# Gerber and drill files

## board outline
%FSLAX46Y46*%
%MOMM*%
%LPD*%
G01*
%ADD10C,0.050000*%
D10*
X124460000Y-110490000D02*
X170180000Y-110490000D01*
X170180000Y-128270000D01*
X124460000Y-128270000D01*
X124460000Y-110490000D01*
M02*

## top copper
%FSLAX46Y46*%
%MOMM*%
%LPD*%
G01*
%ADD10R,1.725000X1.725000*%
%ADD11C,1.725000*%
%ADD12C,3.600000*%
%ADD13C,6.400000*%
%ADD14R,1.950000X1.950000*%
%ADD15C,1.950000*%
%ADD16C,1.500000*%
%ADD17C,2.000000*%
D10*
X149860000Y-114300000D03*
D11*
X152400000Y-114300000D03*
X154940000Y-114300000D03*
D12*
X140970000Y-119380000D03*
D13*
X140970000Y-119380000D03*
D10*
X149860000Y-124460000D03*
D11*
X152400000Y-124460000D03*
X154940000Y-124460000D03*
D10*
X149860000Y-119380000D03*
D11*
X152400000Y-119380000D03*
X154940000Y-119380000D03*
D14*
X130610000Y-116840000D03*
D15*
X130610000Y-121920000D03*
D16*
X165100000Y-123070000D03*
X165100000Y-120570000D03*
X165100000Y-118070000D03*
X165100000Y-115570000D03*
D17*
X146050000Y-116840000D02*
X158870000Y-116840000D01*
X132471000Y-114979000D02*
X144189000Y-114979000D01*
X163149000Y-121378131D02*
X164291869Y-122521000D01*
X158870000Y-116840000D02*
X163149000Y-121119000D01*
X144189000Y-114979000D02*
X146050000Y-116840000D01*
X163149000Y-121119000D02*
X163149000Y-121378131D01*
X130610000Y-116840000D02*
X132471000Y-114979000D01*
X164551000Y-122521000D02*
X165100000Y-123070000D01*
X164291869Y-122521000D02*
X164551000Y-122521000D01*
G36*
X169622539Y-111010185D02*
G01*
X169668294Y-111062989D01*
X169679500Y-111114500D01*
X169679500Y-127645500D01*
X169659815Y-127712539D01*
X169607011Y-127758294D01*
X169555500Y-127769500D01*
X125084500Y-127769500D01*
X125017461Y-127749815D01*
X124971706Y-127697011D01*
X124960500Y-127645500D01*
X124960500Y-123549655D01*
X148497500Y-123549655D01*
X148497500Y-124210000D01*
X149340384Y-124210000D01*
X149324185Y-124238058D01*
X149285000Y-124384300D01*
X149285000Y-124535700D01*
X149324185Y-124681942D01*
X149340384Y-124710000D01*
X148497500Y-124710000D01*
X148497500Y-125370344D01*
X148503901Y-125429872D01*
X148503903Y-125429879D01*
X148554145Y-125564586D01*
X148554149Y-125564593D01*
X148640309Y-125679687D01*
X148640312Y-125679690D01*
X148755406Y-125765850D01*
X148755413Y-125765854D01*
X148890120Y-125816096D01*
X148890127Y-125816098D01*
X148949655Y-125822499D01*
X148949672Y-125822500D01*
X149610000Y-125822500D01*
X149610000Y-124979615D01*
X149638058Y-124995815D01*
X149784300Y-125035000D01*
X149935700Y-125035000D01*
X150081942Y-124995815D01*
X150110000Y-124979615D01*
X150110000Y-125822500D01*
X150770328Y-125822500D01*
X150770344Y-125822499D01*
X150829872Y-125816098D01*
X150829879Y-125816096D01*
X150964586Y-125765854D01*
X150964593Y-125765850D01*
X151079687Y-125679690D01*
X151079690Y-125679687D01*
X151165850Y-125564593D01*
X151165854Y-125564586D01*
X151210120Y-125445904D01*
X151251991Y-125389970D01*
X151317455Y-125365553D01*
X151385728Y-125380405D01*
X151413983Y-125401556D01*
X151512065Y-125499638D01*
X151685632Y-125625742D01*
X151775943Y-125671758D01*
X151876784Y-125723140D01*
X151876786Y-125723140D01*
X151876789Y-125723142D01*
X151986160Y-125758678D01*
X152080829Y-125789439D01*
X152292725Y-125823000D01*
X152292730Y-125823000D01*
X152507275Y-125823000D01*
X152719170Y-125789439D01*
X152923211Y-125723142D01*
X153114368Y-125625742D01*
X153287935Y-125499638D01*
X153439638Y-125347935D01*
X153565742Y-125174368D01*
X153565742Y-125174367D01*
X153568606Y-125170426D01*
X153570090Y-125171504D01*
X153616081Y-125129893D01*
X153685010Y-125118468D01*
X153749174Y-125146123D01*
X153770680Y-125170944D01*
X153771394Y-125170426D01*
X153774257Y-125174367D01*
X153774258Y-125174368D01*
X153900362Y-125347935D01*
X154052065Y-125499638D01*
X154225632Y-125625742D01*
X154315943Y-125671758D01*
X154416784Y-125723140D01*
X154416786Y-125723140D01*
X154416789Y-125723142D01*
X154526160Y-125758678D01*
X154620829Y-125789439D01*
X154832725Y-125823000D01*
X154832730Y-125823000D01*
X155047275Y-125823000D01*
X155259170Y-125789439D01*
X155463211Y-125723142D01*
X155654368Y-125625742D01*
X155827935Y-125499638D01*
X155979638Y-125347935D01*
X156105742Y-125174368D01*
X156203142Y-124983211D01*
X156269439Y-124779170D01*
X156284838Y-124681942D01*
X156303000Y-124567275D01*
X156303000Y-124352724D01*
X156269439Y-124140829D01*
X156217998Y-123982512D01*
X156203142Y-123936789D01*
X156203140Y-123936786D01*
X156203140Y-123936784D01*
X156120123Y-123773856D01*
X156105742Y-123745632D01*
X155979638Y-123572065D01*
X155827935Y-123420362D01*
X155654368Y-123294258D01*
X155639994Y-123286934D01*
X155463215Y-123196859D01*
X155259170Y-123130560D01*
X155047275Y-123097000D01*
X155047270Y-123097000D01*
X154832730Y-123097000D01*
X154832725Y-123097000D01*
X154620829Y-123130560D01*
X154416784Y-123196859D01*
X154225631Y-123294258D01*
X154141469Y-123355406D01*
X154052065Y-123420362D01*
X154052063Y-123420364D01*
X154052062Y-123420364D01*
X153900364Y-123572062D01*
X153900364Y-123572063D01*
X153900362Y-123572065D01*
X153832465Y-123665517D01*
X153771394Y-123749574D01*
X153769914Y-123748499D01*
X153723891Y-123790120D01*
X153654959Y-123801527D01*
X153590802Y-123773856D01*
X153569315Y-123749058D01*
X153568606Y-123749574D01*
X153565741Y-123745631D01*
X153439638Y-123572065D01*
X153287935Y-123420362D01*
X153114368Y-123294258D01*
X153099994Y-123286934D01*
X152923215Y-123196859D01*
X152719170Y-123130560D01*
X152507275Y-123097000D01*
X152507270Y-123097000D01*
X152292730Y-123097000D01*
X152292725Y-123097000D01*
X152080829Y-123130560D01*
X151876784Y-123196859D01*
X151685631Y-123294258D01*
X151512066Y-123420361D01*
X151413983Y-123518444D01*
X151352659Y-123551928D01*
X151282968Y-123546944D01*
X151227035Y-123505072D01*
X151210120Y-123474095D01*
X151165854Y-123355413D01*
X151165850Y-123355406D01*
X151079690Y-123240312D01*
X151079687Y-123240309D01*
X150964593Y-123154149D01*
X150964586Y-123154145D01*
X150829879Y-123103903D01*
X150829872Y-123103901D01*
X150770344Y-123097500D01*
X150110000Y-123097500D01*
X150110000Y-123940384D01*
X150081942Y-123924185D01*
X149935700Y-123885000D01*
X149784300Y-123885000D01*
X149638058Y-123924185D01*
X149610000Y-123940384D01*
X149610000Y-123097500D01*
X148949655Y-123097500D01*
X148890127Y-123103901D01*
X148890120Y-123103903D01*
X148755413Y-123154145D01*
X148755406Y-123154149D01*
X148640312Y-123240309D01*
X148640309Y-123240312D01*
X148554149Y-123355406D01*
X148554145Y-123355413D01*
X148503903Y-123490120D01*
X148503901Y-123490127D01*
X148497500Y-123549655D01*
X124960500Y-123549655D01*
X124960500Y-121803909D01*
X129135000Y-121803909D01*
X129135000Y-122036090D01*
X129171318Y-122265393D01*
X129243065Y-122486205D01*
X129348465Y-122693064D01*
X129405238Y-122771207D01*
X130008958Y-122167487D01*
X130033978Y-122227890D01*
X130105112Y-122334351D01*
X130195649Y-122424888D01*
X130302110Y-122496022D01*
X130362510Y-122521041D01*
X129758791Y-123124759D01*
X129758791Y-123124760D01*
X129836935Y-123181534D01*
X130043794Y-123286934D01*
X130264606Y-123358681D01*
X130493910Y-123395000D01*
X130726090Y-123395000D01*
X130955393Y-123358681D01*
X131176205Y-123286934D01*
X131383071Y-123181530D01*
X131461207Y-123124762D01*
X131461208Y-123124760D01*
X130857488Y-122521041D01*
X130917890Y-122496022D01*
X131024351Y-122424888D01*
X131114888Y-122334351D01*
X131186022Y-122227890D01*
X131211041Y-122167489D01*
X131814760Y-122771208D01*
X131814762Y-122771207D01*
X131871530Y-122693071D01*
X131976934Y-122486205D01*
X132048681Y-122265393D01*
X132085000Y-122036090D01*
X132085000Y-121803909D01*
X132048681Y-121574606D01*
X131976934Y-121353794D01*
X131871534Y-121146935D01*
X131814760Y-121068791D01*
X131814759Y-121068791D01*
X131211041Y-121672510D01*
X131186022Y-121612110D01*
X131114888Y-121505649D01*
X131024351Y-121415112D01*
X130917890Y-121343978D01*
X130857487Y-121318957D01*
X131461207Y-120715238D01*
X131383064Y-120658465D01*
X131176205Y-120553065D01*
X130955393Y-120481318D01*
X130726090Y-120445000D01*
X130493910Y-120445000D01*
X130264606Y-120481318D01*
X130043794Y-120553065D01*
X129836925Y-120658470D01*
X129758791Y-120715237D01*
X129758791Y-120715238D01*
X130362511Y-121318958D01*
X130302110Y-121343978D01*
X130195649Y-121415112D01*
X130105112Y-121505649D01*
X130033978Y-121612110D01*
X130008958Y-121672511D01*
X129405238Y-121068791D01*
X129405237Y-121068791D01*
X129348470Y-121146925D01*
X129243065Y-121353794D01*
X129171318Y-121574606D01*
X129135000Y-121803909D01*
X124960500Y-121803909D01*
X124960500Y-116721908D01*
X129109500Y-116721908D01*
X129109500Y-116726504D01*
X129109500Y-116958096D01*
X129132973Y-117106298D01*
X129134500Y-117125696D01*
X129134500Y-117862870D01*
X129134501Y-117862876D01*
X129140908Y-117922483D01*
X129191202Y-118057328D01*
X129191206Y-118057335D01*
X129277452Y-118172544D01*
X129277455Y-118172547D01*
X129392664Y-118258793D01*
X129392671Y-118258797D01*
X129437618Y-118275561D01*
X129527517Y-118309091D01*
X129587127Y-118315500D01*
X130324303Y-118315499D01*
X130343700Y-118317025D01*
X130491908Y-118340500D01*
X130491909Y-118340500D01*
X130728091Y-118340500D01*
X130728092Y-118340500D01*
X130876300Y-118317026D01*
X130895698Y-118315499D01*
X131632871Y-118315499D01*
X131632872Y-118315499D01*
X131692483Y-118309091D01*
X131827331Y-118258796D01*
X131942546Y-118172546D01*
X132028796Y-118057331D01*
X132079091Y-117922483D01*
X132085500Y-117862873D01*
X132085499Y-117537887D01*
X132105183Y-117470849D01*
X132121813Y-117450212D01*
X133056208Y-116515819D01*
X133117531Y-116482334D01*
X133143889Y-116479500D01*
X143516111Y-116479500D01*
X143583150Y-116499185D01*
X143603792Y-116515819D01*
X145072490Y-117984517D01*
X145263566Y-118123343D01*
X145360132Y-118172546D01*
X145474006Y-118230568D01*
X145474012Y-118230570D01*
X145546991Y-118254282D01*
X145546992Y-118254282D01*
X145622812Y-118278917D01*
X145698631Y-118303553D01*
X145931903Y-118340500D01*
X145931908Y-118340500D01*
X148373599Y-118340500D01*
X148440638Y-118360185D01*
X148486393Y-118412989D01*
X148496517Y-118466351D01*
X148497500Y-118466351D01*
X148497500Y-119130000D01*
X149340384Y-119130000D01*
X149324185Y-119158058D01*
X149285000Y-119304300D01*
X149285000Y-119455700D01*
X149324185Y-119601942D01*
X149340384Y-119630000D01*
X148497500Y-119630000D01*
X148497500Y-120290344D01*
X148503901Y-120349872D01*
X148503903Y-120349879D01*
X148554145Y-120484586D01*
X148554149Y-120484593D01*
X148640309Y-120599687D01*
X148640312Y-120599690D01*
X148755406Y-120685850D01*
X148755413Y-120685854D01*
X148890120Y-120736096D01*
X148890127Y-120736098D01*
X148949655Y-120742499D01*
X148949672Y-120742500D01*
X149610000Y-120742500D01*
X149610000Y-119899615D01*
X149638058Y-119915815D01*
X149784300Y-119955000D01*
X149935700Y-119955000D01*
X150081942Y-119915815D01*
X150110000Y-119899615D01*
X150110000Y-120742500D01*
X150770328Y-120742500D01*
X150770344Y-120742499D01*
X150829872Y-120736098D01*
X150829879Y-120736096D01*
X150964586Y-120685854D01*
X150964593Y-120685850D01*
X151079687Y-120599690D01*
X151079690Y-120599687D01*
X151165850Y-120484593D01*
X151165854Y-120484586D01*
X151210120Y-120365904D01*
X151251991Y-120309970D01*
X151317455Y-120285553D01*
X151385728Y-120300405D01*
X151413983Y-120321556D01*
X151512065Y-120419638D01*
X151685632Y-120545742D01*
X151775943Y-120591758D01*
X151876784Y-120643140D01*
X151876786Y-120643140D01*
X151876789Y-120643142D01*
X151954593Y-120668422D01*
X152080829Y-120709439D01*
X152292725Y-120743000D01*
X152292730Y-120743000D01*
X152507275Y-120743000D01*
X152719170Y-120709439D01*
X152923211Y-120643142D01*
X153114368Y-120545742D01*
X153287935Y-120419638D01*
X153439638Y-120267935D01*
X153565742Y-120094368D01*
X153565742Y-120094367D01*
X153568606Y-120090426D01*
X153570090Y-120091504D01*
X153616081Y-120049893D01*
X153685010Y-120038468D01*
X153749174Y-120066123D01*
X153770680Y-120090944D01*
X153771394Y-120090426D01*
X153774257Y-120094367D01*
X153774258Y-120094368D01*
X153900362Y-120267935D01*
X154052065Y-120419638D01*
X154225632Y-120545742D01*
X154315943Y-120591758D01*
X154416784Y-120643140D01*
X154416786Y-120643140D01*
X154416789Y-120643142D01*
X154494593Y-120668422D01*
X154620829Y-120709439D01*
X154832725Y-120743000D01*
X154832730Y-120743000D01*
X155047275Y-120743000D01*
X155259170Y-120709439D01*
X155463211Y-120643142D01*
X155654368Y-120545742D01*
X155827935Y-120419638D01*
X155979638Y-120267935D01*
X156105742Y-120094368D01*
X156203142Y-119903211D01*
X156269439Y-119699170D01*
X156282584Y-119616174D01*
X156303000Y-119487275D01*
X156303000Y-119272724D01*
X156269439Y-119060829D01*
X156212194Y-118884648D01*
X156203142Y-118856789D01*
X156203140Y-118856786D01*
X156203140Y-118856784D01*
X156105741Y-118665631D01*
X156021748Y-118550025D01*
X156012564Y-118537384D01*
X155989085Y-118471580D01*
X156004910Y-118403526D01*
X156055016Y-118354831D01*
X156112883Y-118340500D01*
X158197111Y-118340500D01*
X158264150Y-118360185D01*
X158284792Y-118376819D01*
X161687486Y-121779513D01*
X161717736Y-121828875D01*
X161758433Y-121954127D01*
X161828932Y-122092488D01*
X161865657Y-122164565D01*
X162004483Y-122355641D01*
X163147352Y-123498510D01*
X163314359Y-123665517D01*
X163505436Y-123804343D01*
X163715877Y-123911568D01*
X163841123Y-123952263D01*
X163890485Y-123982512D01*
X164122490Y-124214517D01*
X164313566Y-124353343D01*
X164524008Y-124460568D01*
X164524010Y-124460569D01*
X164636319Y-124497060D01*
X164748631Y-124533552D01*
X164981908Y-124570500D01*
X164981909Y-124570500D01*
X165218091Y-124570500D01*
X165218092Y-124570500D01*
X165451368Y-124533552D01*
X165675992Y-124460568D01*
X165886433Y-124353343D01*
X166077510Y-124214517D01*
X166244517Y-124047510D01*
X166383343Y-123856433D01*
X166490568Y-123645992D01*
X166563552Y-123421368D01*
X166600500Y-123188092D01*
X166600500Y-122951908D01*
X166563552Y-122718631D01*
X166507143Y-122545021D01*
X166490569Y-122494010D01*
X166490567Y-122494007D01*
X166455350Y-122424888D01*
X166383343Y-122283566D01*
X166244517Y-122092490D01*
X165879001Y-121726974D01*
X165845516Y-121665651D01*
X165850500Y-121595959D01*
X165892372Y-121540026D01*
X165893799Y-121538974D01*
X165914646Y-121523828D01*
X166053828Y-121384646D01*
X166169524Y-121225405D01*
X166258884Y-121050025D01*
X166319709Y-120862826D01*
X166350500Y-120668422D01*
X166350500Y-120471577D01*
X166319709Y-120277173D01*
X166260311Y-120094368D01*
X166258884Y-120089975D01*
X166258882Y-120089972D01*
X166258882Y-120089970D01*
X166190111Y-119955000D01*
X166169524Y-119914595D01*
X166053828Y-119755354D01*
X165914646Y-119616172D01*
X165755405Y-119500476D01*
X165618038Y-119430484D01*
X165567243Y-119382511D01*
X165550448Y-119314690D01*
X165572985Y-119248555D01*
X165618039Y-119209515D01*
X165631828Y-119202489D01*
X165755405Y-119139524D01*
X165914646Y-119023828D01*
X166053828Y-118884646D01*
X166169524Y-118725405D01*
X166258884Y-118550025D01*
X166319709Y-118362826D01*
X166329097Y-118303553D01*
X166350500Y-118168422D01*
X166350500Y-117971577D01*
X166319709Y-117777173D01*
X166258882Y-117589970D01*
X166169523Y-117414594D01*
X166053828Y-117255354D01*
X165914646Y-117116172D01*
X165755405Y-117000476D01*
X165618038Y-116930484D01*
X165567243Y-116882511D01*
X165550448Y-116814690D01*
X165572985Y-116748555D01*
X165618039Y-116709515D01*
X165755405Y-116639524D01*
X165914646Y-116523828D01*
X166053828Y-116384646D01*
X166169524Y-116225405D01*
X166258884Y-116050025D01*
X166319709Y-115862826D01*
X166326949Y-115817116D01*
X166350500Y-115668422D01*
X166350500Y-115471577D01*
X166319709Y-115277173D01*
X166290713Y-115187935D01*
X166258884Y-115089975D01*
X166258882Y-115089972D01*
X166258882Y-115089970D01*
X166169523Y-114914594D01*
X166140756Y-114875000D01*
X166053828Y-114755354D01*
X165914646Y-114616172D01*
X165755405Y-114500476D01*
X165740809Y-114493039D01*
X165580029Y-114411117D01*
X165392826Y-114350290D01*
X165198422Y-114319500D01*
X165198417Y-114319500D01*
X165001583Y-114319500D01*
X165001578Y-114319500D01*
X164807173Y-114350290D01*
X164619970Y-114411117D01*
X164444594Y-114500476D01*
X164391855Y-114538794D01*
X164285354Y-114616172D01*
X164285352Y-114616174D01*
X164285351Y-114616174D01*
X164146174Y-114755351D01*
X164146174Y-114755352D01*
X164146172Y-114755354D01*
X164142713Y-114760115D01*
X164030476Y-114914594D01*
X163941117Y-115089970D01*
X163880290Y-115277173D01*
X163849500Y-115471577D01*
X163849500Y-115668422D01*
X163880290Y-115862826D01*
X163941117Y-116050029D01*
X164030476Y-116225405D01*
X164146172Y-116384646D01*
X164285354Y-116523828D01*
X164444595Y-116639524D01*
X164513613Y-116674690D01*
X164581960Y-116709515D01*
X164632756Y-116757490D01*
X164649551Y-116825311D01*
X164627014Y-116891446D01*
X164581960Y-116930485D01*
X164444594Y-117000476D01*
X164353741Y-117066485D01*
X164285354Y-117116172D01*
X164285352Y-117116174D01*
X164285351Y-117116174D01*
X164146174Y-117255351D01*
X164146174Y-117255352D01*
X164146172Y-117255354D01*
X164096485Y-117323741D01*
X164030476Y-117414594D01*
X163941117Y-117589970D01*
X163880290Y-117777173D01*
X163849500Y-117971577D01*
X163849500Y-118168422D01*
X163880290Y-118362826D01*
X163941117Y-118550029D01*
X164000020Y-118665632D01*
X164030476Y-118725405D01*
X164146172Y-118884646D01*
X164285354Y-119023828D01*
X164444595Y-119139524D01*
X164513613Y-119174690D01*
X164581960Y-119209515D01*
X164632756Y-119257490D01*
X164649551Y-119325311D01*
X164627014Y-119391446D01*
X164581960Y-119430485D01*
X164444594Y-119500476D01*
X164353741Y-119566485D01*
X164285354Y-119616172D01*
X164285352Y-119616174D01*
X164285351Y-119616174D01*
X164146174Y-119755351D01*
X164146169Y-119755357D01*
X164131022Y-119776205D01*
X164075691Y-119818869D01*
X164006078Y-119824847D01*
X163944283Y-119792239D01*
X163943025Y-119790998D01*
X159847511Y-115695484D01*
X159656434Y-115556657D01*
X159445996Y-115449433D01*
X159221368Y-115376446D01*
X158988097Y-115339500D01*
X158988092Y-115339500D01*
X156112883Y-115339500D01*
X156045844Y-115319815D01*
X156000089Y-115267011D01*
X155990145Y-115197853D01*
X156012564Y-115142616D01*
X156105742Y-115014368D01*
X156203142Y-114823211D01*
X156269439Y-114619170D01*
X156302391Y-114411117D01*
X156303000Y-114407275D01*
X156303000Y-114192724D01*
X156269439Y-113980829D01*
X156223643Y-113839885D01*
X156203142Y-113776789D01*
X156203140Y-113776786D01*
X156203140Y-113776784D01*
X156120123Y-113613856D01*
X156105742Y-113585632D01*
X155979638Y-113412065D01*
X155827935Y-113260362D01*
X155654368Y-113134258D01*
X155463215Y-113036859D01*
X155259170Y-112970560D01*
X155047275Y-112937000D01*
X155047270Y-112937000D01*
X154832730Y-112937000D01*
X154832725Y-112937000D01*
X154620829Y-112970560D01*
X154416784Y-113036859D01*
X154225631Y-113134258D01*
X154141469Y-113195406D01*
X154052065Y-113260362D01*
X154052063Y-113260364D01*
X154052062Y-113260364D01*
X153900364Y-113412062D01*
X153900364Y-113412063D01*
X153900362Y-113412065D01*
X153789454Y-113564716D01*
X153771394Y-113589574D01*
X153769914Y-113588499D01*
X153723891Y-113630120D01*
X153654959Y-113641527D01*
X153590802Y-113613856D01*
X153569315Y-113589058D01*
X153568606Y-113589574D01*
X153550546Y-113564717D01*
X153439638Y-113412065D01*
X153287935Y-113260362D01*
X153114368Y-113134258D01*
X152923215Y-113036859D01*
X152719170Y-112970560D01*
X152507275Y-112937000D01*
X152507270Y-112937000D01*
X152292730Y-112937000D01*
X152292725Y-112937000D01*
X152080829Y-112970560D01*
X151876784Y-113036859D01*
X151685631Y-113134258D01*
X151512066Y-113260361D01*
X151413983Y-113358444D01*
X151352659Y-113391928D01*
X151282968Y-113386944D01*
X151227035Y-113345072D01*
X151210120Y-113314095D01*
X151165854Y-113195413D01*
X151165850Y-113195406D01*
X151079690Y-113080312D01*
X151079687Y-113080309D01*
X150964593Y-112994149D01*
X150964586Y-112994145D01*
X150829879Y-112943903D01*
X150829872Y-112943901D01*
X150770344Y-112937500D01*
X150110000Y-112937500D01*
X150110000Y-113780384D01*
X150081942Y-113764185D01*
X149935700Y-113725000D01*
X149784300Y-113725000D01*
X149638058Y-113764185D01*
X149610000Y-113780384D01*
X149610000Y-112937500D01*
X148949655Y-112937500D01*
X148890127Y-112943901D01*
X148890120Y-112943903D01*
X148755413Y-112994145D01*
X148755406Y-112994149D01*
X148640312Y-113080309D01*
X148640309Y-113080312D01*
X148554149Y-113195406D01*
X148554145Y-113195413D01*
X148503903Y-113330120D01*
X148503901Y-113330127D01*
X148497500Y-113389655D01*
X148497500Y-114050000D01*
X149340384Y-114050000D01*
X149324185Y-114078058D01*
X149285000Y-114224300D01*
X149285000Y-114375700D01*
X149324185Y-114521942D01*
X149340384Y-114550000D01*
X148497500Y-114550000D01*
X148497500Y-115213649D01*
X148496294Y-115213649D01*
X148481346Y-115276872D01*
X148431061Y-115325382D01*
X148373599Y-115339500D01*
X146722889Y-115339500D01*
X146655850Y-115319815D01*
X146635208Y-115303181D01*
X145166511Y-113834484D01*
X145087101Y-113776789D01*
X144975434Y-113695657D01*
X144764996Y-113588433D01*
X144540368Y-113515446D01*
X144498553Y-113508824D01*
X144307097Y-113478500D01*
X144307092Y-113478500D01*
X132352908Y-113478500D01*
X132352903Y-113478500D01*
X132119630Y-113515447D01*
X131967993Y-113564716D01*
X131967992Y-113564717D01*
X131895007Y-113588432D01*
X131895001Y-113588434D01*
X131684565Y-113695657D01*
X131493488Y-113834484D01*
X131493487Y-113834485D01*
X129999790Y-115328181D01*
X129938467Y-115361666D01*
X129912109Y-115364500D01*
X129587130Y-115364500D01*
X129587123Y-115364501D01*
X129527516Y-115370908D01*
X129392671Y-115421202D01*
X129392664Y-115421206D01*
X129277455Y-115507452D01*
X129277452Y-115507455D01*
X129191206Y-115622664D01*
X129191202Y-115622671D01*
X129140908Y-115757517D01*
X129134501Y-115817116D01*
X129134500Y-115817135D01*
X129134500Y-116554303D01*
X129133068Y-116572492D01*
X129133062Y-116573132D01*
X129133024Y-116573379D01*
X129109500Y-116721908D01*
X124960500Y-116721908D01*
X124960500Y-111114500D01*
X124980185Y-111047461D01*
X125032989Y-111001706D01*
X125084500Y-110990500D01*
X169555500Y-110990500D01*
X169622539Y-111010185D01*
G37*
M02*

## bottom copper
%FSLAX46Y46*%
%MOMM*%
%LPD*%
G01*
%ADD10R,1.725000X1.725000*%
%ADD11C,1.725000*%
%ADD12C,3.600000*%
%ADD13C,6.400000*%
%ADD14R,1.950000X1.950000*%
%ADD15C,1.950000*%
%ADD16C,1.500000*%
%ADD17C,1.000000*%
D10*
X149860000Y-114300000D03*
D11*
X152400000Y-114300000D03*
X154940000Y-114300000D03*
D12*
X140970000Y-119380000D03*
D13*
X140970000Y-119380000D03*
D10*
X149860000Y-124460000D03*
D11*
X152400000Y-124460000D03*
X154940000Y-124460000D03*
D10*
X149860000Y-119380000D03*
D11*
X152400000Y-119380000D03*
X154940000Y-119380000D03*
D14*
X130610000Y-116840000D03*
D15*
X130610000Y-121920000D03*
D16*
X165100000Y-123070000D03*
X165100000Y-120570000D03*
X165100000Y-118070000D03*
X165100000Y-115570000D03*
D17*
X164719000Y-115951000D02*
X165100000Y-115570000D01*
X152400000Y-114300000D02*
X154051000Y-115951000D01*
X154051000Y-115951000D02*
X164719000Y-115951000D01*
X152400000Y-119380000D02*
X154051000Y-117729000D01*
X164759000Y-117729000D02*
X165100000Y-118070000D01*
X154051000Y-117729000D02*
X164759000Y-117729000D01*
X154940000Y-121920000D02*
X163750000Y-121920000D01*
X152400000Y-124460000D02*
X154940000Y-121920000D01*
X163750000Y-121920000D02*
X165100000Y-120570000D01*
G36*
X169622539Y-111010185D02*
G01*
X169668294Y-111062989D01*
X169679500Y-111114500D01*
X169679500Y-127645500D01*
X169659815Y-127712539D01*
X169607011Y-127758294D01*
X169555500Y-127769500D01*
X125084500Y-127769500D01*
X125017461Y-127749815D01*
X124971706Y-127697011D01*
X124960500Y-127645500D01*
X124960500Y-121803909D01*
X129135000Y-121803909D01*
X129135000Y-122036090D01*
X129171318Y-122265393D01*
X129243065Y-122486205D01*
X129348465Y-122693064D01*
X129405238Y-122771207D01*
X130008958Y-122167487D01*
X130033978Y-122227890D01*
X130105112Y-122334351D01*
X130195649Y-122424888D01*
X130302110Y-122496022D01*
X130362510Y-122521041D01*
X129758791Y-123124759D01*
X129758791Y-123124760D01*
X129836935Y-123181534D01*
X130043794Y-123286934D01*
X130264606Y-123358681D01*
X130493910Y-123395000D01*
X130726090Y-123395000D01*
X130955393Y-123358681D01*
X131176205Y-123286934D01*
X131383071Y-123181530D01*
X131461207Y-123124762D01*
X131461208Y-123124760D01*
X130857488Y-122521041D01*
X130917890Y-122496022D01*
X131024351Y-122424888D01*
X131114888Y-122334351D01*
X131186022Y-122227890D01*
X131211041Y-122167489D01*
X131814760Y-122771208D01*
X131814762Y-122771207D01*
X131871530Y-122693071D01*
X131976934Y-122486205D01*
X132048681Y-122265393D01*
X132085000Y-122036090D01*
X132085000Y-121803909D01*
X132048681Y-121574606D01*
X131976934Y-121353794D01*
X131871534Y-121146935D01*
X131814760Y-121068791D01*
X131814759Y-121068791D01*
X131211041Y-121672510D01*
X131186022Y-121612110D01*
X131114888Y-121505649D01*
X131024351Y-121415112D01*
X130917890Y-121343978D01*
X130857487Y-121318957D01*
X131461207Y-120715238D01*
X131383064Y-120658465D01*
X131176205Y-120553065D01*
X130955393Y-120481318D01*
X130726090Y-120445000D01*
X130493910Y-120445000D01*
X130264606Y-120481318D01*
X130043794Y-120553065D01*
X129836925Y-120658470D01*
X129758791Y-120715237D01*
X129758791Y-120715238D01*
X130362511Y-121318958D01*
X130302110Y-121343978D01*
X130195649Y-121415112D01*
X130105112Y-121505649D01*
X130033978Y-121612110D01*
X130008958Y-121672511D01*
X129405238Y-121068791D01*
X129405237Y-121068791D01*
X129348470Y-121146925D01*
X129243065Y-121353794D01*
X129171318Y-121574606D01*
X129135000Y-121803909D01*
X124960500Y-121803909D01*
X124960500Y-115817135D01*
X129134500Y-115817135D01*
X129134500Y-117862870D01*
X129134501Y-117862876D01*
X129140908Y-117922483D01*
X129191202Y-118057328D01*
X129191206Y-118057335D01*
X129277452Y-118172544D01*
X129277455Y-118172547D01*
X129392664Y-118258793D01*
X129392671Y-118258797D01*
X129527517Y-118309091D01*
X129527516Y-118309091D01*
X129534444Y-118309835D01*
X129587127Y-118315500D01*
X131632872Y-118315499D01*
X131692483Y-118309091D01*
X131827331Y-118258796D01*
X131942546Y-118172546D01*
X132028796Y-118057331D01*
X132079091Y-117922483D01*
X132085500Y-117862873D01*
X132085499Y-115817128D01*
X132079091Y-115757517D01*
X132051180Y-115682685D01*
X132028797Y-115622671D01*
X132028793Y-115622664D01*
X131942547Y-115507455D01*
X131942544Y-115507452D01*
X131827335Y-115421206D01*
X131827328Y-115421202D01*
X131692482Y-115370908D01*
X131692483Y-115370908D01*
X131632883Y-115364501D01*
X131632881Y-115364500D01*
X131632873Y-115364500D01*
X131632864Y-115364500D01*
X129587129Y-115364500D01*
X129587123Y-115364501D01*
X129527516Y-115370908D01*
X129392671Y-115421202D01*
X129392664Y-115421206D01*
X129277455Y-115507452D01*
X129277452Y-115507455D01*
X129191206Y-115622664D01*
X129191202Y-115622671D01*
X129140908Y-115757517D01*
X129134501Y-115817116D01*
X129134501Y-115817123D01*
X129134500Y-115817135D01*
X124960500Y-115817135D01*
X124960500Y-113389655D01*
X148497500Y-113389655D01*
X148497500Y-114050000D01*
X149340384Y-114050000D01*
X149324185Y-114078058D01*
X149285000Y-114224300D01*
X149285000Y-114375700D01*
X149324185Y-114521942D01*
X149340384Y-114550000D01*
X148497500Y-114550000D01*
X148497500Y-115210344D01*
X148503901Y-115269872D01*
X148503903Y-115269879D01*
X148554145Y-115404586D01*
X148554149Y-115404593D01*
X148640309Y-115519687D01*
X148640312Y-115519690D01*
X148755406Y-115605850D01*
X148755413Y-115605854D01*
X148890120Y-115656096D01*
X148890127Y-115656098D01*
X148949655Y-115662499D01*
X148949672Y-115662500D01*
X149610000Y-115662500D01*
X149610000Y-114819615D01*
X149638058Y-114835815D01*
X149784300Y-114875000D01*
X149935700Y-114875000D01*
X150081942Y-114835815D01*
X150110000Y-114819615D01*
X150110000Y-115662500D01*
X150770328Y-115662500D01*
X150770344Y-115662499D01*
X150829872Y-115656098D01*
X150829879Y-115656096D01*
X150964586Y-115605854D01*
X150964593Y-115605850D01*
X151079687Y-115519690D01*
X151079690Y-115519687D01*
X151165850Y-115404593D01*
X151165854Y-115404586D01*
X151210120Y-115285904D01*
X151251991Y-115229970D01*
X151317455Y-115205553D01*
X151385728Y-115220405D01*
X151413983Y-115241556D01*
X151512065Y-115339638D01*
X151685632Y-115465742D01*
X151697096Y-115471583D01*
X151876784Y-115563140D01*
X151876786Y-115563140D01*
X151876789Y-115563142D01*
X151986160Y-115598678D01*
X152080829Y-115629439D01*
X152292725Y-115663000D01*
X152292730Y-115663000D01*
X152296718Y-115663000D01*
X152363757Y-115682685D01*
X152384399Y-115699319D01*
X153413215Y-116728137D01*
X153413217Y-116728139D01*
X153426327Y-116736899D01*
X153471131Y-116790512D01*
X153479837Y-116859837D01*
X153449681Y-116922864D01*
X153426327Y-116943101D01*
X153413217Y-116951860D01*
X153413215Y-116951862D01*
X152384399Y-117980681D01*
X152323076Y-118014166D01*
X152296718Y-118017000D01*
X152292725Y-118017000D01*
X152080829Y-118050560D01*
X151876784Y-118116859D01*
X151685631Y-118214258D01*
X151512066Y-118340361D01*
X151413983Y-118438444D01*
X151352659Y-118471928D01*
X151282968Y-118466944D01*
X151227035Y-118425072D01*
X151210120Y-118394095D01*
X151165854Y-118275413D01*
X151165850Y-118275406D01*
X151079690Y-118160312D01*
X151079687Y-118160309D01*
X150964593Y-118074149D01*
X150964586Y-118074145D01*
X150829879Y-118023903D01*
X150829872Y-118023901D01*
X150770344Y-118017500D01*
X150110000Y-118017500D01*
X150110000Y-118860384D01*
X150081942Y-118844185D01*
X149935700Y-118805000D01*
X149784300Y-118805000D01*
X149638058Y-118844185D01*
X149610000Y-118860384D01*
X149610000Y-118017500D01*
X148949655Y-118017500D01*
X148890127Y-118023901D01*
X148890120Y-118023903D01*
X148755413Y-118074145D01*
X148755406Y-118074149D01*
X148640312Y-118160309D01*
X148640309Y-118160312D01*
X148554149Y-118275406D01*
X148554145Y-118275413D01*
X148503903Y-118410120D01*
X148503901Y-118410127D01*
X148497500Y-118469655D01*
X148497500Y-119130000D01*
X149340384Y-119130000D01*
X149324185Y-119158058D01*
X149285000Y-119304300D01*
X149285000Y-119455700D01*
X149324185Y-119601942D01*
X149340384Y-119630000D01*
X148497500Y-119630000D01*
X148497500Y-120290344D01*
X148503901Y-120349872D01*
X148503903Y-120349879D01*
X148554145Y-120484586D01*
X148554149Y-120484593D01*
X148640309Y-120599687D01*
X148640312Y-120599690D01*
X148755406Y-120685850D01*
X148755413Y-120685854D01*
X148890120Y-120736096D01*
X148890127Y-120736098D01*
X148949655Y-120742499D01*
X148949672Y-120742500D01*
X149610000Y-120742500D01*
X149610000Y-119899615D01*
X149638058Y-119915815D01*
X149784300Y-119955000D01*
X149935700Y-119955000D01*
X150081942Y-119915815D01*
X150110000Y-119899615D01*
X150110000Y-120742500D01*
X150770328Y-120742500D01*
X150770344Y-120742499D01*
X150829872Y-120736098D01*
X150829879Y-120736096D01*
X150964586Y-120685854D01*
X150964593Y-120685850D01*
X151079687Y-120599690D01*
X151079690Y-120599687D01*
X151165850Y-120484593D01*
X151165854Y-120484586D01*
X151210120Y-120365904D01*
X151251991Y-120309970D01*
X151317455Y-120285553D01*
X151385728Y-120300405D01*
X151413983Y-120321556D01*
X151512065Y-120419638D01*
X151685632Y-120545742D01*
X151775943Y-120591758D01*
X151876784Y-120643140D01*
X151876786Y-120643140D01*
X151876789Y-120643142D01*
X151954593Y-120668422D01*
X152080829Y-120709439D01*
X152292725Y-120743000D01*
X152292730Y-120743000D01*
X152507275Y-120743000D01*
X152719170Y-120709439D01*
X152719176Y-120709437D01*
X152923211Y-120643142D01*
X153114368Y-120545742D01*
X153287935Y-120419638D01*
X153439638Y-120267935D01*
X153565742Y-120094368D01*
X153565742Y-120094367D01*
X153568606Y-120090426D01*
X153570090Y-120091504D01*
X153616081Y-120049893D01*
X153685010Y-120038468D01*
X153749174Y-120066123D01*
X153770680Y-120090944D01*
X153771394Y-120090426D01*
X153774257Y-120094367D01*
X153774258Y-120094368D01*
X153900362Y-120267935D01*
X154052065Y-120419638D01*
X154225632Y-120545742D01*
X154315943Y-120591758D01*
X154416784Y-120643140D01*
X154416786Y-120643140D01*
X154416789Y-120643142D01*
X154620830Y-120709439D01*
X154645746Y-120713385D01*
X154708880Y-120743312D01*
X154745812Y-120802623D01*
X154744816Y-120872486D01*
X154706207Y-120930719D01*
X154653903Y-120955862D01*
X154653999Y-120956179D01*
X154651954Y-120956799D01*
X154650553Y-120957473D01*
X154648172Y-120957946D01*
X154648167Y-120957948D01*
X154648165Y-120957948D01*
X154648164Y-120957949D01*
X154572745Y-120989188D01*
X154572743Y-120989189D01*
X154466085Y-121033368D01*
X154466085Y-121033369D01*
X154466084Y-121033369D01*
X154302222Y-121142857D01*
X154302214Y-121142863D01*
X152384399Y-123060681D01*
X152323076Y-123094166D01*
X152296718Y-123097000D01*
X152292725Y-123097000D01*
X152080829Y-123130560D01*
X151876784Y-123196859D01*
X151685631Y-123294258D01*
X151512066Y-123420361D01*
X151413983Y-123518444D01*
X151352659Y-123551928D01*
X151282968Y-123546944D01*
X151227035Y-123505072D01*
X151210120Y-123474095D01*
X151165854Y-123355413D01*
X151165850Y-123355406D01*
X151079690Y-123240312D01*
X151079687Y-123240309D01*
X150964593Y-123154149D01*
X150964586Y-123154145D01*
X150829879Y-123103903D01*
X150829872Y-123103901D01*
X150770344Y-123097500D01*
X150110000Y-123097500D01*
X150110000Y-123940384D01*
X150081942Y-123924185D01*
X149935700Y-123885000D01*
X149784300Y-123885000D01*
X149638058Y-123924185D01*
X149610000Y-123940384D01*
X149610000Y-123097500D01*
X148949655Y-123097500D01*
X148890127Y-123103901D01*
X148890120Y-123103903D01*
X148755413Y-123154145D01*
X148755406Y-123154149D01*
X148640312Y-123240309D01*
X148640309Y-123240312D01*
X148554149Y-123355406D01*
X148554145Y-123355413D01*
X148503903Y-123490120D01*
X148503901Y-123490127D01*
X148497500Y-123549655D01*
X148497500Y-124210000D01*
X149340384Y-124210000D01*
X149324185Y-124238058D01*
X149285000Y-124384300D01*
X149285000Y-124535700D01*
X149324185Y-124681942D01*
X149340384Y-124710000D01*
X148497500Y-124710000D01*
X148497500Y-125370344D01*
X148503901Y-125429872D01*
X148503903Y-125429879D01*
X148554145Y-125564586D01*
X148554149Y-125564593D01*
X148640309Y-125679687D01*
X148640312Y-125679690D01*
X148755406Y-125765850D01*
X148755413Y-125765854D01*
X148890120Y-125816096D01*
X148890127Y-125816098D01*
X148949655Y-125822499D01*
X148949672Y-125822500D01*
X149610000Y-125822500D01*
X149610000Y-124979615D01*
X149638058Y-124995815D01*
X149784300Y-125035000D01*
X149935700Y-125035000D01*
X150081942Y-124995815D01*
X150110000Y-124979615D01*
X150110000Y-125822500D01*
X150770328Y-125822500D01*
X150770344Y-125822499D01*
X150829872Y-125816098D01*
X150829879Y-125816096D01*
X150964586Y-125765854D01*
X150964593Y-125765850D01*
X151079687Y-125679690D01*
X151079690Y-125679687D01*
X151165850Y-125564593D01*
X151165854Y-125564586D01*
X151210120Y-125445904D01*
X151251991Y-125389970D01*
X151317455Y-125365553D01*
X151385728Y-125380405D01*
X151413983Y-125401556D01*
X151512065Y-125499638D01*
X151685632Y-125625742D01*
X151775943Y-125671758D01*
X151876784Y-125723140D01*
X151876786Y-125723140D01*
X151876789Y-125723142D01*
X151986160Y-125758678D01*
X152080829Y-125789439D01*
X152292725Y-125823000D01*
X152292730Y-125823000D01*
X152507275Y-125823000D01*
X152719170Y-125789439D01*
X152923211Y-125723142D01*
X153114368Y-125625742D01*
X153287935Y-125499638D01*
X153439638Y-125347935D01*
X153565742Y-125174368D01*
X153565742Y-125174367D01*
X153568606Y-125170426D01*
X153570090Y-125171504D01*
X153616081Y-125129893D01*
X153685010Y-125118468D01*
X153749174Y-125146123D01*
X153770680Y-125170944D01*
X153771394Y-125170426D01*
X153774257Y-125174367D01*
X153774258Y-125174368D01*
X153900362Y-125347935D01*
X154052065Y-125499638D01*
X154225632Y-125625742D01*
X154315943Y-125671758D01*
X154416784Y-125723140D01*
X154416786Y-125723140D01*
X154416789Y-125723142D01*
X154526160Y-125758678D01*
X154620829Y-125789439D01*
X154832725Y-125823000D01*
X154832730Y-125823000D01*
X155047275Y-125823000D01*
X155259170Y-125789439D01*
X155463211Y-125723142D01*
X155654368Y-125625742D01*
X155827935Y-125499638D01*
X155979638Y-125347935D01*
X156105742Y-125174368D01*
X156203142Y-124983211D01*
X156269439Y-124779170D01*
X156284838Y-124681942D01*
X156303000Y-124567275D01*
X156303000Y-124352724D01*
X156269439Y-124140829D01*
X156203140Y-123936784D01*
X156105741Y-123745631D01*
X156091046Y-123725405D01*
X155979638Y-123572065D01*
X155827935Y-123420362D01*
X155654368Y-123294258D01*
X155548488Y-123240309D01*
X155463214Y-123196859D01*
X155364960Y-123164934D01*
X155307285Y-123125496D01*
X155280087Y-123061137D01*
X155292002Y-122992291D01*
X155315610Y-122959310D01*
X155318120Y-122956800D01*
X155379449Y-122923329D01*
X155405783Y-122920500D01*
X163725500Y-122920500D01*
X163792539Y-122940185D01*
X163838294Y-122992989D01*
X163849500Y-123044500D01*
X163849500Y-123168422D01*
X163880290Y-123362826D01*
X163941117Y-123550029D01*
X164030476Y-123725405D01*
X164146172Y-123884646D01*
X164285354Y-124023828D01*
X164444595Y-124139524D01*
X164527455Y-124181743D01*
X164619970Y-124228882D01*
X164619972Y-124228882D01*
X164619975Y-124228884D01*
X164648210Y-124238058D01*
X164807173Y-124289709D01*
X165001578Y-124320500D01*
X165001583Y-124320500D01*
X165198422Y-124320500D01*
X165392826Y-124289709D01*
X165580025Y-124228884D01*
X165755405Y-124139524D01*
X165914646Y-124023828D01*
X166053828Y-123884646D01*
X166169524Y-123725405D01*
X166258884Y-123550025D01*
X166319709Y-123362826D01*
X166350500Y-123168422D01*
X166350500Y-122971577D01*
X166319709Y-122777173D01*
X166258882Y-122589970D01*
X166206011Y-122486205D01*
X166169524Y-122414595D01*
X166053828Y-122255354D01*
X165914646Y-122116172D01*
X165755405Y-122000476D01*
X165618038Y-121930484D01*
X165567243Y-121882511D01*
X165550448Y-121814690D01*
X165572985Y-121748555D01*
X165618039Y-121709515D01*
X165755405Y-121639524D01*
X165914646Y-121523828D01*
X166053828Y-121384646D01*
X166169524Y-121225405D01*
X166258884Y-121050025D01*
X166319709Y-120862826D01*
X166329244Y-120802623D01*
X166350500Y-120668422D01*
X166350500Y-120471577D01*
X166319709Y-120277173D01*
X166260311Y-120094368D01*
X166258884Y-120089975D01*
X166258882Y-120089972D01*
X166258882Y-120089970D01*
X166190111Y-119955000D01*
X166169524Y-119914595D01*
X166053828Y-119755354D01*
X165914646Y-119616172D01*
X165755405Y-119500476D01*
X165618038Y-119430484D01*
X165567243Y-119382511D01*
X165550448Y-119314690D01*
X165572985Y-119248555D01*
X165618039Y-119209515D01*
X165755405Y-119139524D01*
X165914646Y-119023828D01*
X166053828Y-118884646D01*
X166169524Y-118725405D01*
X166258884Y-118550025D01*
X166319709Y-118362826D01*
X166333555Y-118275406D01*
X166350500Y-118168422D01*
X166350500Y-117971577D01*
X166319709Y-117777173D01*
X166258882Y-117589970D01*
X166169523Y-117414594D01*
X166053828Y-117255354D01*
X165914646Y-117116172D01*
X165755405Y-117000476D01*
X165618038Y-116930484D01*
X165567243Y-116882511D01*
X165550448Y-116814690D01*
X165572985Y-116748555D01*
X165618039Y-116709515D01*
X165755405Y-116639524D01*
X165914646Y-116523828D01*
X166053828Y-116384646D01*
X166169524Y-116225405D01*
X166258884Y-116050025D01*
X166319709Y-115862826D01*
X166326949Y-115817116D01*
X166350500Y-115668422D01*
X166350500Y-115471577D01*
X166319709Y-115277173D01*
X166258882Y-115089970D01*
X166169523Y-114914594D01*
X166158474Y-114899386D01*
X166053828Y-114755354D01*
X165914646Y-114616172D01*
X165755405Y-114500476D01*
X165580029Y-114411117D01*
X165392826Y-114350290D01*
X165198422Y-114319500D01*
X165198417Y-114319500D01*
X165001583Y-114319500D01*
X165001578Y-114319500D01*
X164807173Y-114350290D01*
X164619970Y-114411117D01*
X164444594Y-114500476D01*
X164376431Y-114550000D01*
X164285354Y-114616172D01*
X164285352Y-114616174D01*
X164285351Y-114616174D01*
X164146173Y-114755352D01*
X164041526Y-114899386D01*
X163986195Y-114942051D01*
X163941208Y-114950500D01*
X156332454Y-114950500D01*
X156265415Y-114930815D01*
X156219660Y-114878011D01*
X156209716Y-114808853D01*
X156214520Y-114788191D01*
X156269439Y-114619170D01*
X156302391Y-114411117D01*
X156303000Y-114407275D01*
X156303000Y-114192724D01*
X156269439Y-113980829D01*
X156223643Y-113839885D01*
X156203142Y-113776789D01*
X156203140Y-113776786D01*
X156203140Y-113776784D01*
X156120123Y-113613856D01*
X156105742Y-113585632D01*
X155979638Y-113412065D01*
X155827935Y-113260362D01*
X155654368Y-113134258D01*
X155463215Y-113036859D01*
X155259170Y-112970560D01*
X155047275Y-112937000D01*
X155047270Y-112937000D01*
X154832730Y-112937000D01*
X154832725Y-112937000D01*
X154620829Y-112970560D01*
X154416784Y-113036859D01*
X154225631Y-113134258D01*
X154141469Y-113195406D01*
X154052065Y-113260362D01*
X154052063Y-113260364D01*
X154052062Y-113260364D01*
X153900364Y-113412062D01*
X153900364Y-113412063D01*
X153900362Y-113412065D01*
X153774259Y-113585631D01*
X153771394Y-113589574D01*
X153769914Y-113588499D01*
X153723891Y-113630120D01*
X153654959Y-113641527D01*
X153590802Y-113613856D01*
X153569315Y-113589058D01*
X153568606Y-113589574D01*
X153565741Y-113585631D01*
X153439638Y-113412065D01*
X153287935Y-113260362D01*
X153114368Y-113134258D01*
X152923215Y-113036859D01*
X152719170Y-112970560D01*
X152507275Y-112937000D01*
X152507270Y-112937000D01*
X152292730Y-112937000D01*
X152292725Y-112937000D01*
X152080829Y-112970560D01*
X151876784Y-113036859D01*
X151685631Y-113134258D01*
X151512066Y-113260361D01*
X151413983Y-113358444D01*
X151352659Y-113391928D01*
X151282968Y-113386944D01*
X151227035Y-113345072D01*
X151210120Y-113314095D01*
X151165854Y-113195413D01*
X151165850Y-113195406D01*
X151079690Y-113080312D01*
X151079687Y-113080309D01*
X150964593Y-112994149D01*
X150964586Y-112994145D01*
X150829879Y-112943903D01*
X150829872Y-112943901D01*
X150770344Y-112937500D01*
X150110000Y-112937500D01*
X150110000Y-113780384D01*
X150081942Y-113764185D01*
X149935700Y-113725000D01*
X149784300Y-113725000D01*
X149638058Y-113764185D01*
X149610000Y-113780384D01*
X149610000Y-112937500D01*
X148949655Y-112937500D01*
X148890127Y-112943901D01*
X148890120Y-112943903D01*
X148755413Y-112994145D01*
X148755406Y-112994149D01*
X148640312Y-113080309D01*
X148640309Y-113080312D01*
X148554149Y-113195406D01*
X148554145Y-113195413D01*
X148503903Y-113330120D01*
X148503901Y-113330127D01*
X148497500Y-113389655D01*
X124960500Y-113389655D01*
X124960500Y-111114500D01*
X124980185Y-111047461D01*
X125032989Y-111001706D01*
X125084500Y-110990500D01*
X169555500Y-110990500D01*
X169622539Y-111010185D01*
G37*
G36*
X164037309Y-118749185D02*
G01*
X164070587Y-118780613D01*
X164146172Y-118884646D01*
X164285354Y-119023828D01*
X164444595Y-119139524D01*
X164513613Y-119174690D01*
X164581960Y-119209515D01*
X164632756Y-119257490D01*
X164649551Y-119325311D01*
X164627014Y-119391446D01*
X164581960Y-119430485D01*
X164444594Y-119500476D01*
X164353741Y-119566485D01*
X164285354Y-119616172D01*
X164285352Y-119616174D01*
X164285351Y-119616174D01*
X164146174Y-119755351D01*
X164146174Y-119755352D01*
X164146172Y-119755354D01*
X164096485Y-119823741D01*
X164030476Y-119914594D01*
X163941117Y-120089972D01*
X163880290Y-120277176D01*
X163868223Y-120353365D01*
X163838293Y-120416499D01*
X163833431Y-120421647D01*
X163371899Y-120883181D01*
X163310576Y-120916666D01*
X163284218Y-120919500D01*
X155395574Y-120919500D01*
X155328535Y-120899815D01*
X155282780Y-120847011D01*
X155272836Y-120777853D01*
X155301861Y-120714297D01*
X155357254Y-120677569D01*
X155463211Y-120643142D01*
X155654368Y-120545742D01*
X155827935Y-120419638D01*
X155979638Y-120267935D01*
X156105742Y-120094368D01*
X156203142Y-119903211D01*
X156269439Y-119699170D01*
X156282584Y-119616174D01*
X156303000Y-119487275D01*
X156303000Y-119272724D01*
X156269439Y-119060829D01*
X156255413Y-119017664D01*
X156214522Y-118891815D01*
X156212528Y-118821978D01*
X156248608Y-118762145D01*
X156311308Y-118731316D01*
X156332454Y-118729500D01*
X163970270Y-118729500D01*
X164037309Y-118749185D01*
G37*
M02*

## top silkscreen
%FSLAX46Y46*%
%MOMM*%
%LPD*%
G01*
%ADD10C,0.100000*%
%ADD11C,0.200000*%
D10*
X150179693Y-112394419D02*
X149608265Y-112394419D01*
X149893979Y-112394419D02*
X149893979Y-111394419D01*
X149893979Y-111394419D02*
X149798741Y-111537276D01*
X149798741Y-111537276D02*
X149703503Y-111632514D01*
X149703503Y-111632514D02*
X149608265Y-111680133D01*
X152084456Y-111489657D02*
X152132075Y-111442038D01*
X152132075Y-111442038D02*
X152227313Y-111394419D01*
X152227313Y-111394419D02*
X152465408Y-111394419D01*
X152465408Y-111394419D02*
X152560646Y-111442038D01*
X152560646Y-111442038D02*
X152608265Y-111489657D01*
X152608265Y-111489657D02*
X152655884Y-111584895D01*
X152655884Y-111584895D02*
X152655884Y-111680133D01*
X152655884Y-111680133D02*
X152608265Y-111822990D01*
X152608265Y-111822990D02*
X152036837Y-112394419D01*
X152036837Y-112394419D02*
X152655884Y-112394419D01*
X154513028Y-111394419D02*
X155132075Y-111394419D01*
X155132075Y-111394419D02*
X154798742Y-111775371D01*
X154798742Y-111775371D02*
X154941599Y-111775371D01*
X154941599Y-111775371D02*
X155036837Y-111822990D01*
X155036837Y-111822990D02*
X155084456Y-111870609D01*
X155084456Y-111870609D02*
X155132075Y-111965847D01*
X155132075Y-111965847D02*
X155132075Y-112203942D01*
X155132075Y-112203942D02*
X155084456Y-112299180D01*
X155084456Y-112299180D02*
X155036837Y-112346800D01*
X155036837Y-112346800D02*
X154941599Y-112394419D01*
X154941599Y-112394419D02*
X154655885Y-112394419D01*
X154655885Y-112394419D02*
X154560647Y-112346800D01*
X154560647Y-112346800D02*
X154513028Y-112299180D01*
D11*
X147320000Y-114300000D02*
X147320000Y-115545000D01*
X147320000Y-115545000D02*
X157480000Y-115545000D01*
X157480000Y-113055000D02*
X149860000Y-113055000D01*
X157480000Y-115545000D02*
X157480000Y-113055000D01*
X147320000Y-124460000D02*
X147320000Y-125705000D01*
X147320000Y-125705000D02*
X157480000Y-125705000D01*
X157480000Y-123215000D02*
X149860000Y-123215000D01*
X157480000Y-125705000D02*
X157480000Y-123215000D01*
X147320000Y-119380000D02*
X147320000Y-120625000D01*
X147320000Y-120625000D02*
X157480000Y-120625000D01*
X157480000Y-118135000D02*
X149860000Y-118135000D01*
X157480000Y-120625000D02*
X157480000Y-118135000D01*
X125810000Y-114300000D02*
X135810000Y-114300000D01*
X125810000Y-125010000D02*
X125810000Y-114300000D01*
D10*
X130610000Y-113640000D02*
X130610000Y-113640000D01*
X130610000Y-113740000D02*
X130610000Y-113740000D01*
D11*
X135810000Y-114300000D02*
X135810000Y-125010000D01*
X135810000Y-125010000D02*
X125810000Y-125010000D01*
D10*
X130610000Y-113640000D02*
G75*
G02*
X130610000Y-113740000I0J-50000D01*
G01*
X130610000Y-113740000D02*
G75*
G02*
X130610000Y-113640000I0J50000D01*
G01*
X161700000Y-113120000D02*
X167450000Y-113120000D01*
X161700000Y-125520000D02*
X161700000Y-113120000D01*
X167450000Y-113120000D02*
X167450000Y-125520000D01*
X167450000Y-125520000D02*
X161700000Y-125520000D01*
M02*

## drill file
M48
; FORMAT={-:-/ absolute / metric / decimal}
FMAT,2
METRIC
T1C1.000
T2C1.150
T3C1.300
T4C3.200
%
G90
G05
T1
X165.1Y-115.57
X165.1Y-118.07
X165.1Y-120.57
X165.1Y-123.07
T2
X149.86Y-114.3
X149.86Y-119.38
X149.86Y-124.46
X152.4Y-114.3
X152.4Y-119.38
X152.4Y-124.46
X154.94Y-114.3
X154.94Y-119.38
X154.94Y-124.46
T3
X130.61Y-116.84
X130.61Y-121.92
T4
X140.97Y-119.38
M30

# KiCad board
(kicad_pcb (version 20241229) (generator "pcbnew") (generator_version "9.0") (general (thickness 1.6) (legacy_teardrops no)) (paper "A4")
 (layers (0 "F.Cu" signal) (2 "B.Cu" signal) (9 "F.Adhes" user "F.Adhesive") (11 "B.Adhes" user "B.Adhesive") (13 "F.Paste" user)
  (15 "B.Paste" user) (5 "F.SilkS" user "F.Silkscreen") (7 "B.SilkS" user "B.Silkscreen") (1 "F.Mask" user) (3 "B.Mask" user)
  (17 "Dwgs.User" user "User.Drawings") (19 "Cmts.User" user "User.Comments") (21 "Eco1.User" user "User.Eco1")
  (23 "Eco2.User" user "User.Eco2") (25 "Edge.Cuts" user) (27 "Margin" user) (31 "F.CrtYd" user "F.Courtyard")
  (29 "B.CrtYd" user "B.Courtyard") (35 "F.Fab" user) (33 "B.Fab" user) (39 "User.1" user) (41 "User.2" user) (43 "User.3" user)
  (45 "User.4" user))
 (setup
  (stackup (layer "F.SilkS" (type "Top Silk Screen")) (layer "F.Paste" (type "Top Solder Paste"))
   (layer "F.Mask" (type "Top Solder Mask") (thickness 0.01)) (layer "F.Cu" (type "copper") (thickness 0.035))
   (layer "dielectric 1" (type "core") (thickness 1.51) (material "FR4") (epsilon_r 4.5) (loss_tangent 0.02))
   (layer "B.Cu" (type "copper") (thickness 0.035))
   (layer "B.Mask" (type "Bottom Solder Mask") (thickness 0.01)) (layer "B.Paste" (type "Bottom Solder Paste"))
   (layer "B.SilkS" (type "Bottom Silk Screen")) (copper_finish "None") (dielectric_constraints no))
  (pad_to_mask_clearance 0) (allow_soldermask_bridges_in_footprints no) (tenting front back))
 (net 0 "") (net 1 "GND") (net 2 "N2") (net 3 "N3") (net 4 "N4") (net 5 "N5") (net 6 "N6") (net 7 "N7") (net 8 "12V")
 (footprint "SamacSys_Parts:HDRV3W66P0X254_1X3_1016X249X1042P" (layer "F.Cu") (at 149.86 114.3)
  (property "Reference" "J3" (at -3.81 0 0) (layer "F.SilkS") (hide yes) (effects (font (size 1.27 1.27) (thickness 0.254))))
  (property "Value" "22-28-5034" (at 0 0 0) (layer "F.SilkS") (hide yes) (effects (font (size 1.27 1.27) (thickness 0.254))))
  (fp_line (start -2.54 0) (end -2.54 1.245) (stroke (width 0.2) (type solid)) (layer "F.SilkS"))
  (fp_line (start -2.54 1.245) (end 7.62 1.245) (stroke (width 0.2) (type solid)) (layer "F.SilkS"))
  (fp_line (start 7.62 -1.245) (end 0 -1.245) (stroke (width 0.2) (type solid)) (layer "F.SilkS"))
  (fp_line (start 7.62 1.245) (end 7.62 -1.245) (stroke (width 0.2) (type solid)) (layer "F.SilkS"))
  (pad "1" thru_hole rect (at 0 0) (size 1.725 1.725) (drill 1.15) (layers "*.Cu" "*.Mask") (remove_unused_layers no) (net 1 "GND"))
  (pad "2" thru_hole circle (at 2.54 0) (size 1.725 1.725) (drill 1.15) (layers "*.Cu" "*.Mask") (remove_unused_layers no) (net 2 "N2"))
  (pad "3" thru_hole circle (at 5.08 0) (size 1.725 1.725) (drill 1.15) (layers "*.Cu" "*.Mask") (remove_unused_layers no) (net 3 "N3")))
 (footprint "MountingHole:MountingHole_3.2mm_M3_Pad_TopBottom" (layer "F.Cu") (at 140.97 119.38)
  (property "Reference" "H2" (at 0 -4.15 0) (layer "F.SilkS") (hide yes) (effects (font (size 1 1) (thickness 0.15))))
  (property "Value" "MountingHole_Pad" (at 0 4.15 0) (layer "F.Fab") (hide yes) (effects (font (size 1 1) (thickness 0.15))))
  (pad "1" thru_hole circle (at 0 0) (size 3.6 3.6) (drill 3.2) (layers "*.Cu" "*.Mask") (remove_unused_layers no) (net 1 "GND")
   (zone_connect 2))
  (pad "1" connect circle (at 0 0) (size 6.4 6.4) (layers "F.Cu" "F.Mask") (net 1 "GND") (zone_connect 2))
  (pad "1" connect circle (at 0 0) (size 6.4 6.4) (layers "B.Cu" "B.Mask") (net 1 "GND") (zone_connect 2)))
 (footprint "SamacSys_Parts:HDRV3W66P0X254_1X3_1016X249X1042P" (layer "F.Cu") (at 149.86 124.46)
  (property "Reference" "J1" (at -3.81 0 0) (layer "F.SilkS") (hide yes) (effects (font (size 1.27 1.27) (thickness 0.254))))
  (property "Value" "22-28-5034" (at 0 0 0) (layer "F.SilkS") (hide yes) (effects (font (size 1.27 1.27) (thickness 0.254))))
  (fp_line (start -2.54 0) (end -2.54 1.245) (stroke (width 0.2) (type solid)) (layer "F.SilkS"))
  (fp_line (start -2.54 1.245) (end 7.62 1.245) (stroke (width 0.2) (type solid)) (layer "F.SilkS"))
  (fp_line (start 7.62 -1.245) (end 0 -1.245) (stroke (width 0.2) (type solid)) (layer "F.SilkS"))
  (fp_line (start 7.62 1.245) (end 7.62 -1.245) (stroke (width 0.2) (type solid)) (layer "F.SilkS"))
  (pad "1" thru_hole rect (at 0 0) (size 1.725 1.725) (drill 1.15) (layers "*.Cu" "*.Mask") (remove_unused_layers no) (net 1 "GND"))
  (pad "2" thru_hole circle (at 2.54 0) (size 1.725 1.725) (drill 1.15) (layers "*.Cu" "*.Mask") (remove_unused_layers no) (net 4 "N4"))
  (pad "3" thru_hole circle (at 5.08 0) (size 1.725 1.725) (drill 1.15) (layers "*.Cu" "*.Mask") (remove_unused_layers no) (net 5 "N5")))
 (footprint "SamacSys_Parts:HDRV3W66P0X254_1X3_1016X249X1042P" (layer "F.Cu") (at 149.86 119.38)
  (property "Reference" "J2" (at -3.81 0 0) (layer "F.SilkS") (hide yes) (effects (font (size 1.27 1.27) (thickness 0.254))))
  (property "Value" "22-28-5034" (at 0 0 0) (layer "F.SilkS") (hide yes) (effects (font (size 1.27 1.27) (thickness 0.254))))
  (fp_line (start -2.54 0) (end -2.54 1.245) (stroke (width 0.2) (type solid)) (layer "F.SilkS"))
  (fp_line (start -2.54 1.245) (end 7.62 1.245) (stroke (width 0.2) (type solid)) (layer "F.SilkS"))
  (fp_line (start 7.62 -1.245) (end 0 -1.245) (stroke (width 0.2) (type solid)) (layer "F.SilkS"))
  (fp_line (start 7.62 1.245) (end 7.62 -1.245) (stroke (width 0.2) (type solid)) (layer "F.SilkS"))
  (pad "1" thru_hole rect (at 0 0) (size 1.725 1.725) (drill 1.15) (layers "*.Cu" "*.Mask") (remove_unused_layers no) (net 1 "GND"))
  (pad "2" thru_hole circle (at 2.54 0) (size 1.725 1.725) (drill 1.15) (layers "*.Cu" "*.Mask") (remove_unused_layers no) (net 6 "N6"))
  (pad "3" thru_hole circle (at 5.08 0) (size 1.725 1.725) (drill 1.15) (layers "*.Cu" "*.Mask") (remove_unused_layers no) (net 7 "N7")))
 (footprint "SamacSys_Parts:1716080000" (layer "F.Cu") (at 130.61 116.84 -90)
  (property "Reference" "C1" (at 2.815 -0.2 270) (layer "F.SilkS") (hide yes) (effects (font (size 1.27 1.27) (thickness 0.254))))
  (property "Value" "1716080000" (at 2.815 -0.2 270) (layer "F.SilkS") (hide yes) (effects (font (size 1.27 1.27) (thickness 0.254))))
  (fp_line (start -2.54 4.8) (end -2.54 -5.2) (stroke (width 0.2) (type solid)) (layer "F.SilkS"))
  (fp_line (start 8.17 4.8) (end -2.54 4.8) (stroke (width 0.2) (type solid)) (layer "F.SilkS"))
  (fp_line (start -3.2 0) (end -3.2 0) (stroke (width 0.1) (type solid)) (layer "F.SilkS"))
  (fp_line (start -3.1 0) (end -3.1 0) (stroke (width 0.1) (type solid)) (layer "F.SilkS"))
  (fp_line (start -2.54 -5.2) (end 8.17 -5.2) (stroke (width 0.2) (type solid)) (layer "F.SilkS"))
  (fp_line (start 8.17 -5.2) (end 8.17 4.8) (stroke (width 0.2) (type solid)) (layer "F.SilkS"))
  (fp_arc (start -3.2 0) (mid -3.15 -0.05) (end -3.1 0) (stroke (width 0.1) (type solid)) (layer "F.SilkS"))
  (fp_arc (start -3.1 0) (mid -3.15 0.05) (end -3.2 0) (stroke (width 0.1) (type solid)) (layer "F.SilkS"))
  (pad "1" thru_hole rect (at 0 0 270) (size 1.95 1.95) (drill 1.3) (layers "*.Cu" "*.Mask") (remove_unused_layers no) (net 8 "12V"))
  (pad "2" thru_hole circle (at 5.08 0 270) (size 1.95 1.95) (drill 1.3) (layers "*.Cu" "*.Mask") (remove_unused_layers no) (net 1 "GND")))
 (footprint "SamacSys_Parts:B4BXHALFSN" (layer "F.Cu") (at 165.1 123.07 90)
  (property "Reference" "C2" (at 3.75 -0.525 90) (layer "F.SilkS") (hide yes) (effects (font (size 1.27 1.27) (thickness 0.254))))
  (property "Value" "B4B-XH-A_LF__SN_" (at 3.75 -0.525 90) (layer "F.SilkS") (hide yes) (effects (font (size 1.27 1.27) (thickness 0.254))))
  (fp_line (start 9.95 -3.4) (end 9.95 2.35) (stroke (width 0.1) (type solid)) (layer "F.SilkS"))
  (fp_line (start -2.45 -3.4) (end 9.95 -3.4) (stroke (width 0.1) (type solid)) (layer "F.SilkS"))
  (fp_line (start 9.95 2.35) (end -2.45 2.35) (stroke (width 0.1) (type solid)) (layer "F.SilkS"))
  (fp_line (start -2.45 2.35) (end -2.45 -3.4) (stroke (width 0.1) (type solid)) (layer "F.SilkS"))
  (pad "1" thru_hole circle (at 0 0 90) (size 1.5 1.5) (drill 1) (layers "*.Cu" "*.Mask") (remove_unused_layers no) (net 8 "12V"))
  (pad "2" thru_hole circle (at 2.5 0 90) (size 1.5 1.5) (drill 1) (layers "*.Cu" "*.Mask") (remove_unused_layers no) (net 4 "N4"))
  (pad "3" thru_hole circle (at 5 0 90) (size 1.5 1.5) (drill 1) (layers "*.Cu" "*.Mask") (remove_unused_layers no) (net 6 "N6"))
  (pad "4" thru_hole circle (at 7.5 0 90) (size 1.5 1.5) (drill 1) (layers "*.Cu" "*.Mask") (remove_unused_layers no) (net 2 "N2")))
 (gr_rect (start 124.46 110.49) (end 170.18 128.27) (stroke (width 0.05) (type default)) (fill no) (layer "Edge.Cuts"))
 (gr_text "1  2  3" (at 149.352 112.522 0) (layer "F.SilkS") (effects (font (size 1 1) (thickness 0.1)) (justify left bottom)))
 (segment (start 164.719 115.951) (end 165.1 115.57) (width 1) (layer "B.Cu") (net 2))
 (segment (start 152.4 114.3) (end 154.051 115.951) (width 1) (layer "B.Cu") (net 2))
 (segment (start 154.051 115.951) (end 164.719 115.951) (width 1) (layer "B.Cu") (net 2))
 (segment (start 152.4 119.38) (end 154.051 117.729) (width 1) (layer "B.Cu") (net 6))
 (segment (start 164.759 117.729) (end 165.1 118.07) (width 1) (layer "B.Cu") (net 6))
 (segment (start 154.051 117.729) (end 164.759 117.729) (width 1) (layer "B.Cu") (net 6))
 (segment (start 154.94 121.92) (end 163.75 121.92) (width 1) (layer "B.Cu") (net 4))
 (segment (start 152.4 124.46) (end 154.94 121.92) (width 1) (layer "B.Cu") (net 4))
 (segment (start 163.75 121.92) (end 165.1 120.57) (width 1) (layer "B.Cu") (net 4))
 (segment (start 146.05 116.84) (end 158.87 116.84) (width 2) (layer "F.Cu") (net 8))
 (segment (start 132.471 114.979) (end 144.189 114.979) (width 2) (layer "F.Cu") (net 8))
 (segment (start 163.149 121.378131) (end 164.291869 122.521) (width 2) (layer "F.Cu") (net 8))
 (segment (start 158.87 116.84) (end 163.149 121.119) (width 2) (layer "F.Cu") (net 8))
 (segment (start 144.189 114.979) (end 146.05 116.84) (width 2) (layer "F.Cu") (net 8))
 (segment (start 163.149 121.119) (end 163.149 121.378131) (width 2) (layer "F.Cu") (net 8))
 (segment (start 130.61 116.84) (end 132.471 114.979) (width 2) (layer "F.Cu") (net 8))
 (segment (start 164.551 122.521) (end 165.1 123.07) (width 2) (layer "F.Cu") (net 8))
 (segment (start 164.291869 122.521) (end 164.551 122.521) (width 2) (layer "F.Cu") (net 8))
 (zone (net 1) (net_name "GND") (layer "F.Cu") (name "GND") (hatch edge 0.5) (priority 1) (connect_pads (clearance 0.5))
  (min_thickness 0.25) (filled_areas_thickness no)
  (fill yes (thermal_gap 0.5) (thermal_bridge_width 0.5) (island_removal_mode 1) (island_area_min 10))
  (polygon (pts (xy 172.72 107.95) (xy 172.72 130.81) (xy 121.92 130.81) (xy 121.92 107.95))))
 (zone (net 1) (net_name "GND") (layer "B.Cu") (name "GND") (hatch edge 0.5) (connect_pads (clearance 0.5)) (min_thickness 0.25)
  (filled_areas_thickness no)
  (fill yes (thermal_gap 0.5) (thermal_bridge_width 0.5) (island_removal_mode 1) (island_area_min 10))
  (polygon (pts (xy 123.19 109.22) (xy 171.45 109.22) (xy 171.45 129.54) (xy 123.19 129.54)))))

